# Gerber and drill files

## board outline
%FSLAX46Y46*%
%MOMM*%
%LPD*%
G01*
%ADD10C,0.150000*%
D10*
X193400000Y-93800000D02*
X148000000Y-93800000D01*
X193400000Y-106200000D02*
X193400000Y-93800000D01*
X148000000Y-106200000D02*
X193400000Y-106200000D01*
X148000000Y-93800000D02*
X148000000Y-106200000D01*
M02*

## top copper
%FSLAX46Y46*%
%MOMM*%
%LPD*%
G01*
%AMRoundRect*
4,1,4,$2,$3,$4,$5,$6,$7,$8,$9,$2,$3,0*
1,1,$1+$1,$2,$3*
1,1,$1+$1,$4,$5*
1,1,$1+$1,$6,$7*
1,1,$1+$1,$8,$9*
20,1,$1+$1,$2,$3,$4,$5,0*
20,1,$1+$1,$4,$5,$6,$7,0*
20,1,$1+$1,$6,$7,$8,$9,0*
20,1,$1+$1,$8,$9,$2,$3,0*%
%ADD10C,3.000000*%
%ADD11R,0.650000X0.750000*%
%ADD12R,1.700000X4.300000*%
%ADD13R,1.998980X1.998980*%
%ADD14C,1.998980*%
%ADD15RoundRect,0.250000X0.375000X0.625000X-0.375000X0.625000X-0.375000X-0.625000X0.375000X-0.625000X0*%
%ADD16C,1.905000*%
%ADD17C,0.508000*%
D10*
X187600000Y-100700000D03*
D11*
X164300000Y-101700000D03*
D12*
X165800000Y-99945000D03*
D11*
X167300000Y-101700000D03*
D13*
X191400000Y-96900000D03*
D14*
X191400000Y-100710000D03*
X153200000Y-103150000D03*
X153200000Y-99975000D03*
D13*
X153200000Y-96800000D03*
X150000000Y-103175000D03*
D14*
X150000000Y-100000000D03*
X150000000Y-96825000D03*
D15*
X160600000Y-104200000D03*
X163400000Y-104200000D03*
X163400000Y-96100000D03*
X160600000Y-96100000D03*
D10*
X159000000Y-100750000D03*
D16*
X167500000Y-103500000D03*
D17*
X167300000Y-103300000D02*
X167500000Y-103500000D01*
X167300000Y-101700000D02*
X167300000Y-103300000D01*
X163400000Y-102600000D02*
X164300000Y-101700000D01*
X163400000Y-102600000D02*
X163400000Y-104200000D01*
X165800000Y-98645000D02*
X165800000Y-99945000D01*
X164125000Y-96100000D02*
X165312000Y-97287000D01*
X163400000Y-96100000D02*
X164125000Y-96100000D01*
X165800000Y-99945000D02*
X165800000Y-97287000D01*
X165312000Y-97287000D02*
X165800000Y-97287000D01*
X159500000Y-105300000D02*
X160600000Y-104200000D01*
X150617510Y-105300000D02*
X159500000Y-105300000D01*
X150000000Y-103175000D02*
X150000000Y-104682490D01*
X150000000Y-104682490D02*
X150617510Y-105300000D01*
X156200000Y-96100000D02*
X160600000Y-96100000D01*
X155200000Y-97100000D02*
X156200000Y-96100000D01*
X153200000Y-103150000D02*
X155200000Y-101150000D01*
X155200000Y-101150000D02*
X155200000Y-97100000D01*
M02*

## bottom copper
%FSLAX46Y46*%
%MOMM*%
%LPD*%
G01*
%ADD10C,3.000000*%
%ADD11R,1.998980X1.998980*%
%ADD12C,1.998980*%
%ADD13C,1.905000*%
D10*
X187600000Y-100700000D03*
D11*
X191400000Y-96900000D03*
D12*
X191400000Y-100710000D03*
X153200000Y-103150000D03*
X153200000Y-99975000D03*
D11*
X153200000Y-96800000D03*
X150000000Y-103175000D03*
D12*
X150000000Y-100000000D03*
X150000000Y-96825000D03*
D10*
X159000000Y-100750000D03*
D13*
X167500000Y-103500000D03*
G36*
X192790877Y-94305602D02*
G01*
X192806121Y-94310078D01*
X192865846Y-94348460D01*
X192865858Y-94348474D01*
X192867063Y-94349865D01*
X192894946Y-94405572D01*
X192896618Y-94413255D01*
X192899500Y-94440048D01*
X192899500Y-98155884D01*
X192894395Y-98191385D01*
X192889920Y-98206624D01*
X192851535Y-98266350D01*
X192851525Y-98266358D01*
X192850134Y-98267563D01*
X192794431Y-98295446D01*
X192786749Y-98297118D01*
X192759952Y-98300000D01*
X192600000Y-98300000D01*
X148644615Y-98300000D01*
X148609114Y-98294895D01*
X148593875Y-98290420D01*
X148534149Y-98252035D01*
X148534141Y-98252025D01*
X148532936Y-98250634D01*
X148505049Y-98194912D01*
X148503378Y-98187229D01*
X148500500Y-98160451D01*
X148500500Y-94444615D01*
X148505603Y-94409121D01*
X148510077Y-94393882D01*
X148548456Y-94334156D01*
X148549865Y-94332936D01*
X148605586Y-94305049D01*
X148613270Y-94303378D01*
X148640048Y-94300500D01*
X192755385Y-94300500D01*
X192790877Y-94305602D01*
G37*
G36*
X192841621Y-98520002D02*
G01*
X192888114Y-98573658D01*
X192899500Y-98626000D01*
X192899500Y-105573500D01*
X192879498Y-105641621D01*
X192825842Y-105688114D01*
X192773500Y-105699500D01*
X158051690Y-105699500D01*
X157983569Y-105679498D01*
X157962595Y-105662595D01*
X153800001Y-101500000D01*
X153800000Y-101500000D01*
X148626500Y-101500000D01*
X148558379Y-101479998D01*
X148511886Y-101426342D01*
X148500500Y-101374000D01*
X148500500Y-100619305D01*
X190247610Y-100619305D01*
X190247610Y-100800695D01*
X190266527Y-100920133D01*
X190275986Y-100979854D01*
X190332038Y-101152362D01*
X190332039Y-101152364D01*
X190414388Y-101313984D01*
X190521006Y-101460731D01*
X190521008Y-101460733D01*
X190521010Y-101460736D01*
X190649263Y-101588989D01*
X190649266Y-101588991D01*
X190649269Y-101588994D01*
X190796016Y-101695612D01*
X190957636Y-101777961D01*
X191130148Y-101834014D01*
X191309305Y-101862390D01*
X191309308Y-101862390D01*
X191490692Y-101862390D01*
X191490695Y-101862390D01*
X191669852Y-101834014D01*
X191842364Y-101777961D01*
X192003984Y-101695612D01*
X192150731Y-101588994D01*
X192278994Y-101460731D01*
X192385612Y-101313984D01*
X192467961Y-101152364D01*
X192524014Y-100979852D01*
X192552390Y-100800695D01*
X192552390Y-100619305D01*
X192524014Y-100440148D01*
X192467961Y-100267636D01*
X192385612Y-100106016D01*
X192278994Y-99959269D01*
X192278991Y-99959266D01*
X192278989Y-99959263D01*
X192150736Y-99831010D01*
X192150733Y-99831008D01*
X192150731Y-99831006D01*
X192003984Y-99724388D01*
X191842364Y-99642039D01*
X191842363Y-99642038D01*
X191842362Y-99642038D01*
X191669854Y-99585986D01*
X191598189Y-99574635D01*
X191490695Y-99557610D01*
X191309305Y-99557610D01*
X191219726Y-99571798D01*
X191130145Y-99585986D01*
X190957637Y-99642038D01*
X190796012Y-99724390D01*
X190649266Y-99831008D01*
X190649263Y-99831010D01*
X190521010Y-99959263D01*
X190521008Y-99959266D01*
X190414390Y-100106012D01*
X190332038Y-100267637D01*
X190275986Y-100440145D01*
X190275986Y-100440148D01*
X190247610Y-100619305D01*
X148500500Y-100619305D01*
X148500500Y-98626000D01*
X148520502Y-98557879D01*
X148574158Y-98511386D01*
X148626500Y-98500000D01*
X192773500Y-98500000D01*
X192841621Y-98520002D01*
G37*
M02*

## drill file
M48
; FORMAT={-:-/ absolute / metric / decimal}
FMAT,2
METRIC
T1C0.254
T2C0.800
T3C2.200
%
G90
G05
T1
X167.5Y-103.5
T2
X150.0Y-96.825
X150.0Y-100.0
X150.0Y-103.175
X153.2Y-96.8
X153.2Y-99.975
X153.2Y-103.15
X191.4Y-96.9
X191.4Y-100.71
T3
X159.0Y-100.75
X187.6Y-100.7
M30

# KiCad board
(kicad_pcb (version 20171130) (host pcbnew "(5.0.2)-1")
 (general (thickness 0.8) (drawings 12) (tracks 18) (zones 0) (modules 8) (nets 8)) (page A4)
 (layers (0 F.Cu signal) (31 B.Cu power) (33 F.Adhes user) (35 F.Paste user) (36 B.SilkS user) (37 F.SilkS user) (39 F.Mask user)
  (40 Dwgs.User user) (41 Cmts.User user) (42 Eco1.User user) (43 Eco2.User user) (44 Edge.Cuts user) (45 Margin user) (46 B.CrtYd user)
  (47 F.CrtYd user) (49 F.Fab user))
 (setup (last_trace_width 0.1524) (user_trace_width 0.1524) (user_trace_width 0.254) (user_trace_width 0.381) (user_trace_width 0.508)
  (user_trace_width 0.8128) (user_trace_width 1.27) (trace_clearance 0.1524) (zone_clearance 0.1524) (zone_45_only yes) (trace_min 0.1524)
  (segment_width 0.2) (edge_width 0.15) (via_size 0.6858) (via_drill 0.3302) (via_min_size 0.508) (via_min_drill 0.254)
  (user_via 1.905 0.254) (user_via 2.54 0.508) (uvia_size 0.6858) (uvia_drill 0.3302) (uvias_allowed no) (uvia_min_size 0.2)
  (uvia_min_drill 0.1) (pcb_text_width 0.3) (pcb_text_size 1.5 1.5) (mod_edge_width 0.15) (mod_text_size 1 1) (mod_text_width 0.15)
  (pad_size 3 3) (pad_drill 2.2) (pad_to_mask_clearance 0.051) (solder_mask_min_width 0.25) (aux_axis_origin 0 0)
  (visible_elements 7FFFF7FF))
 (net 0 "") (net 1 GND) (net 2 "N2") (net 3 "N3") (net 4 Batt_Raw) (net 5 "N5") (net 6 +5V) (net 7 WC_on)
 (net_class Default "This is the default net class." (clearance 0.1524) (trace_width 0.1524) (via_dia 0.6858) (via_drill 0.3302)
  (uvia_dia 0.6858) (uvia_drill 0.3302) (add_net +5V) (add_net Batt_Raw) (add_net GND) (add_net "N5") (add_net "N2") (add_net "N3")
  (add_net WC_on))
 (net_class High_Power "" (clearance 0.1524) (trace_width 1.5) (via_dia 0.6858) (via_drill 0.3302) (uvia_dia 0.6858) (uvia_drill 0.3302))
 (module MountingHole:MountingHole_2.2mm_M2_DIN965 (layer F.Cu) (at 187.6 100.7)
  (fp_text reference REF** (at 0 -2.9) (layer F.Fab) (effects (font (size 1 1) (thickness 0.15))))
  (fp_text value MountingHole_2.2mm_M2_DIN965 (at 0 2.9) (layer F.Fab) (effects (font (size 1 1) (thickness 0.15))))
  (pad "" thru_hole circle (at 0 0) (size 3 3) (drill 2.2) (layers *.Cu *.Mask) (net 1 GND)))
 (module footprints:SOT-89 (layer F.Cu) (at 165.8 101.7)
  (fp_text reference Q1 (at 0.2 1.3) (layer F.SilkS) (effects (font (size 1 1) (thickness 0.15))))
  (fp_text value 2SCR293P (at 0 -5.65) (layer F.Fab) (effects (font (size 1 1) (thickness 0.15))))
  (pad 1 smd rect (at -1.5 0) (size 0.65 0.75) (layers F.Cu F.Paste F.Mask) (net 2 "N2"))
  (pad 2 smd rect (at 0 -1.755) (size 1.7 4.3) (layers F.Cu F.Paste F.Mask) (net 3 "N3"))
  (pad 3 smd rect (at 1.5 0) (size 0.65 0.75) (layers F.Cu F.Paste F.Mask) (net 1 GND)))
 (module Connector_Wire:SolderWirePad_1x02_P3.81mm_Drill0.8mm (layer F.Cu) (at 191.4 96.9 270)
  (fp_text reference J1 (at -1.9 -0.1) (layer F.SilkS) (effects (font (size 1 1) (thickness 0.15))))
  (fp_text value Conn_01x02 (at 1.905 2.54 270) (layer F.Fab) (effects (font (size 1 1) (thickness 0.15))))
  (pad 1 thru_hole rect (at 0 0 270) (size 1.99898 1.99898) (drill 0.8001) (layers *.Cu *.Mask) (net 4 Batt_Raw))
  (pad 2 thru_hole circle (at 3.81 0 270) (size 1.99898 1.99898) (drill 0.8001) (layers *.Cu *.Mask) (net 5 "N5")))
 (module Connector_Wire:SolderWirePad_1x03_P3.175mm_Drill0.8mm (layer F.Cu) (at 153.2 96.8 270)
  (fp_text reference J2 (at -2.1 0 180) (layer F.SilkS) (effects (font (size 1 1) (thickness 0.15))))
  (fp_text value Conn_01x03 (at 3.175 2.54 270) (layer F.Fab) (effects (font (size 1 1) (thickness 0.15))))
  (pad 3 thru_hole circle (at 6.35 0 270) (size 1.99898 1.99898) (drill 0.8001) (layers *.Cu *.Mask) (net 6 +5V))
  (pad 2 thru_hole circle (at 3.175 0 270) (size 1.99898 1.99898) (drill 0.8001) (layers *.Cu *.Mask) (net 1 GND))
  (pad 1 thru_hole rect (at 0 0 270) (size 1.99898 1.99898) (drill 0.8001) (layers *.Cu *.Mask) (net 4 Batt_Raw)))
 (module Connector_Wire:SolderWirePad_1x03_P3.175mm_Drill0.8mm (layer F.Cu) (at 150 103.175 90)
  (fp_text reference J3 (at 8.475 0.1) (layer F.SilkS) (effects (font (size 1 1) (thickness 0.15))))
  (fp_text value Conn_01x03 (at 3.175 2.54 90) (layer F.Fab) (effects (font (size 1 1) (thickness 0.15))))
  (pad 1 thru_hole rect (at 0 0 90) (size 1.99898 1.99898) (drill 0.8001) (layers *.Cu *.Mask) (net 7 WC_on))
  (pad 2 thru_hole circle (at 3.175 0 90) (size 1.99898 1.99898) (drill 0.8001) (layers *.Cu *.Mask) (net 1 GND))
  (pad 3 thru_hole circle (at 6.35 0 90) (size 1.99898 1.99898) (drill 0.8001) (layers *.Cu *.Mask) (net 4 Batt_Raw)))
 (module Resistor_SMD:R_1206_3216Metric (layer F.Cu) (at 162 104.2 180)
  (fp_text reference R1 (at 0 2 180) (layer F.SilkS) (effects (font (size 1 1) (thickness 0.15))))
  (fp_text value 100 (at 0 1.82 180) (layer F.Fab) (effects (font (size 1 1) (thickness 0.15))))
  (pad 2 smd roundrect (at 1.4 0 180) (size 1.25 1.75) (layers F.Cu F.Paste F.Mask) (roundrect_rratio 0.2) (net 7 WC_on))
  (pad 1 smd roundrect (at -1.4 0 180) (size 1.25 1.75) (layers F.Cu F.Paste F.Mask) (roundrect_rratio 0.2) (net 2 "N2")))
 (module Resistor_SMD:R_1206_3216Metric (layer F.Cu) (at 162 96.1 180)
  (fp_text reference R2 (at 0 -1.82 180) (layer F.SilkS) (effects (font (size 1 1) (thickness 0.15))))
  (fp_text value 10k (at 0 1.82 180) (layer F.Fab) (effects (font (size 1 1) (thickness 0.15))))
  (pad 1 smd roundrect (at -1.4 0 180) (size 1.25 1.75) (layers F.Cu F.Paste F.Mask) (roundrect_rratio 0.2) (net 3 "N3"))
  (pad 2 smd roundrect (at 1.4 0 180) (size 1.25 1.75) (layers F.Cu F.Paste F.Mask) (roundrect_rratio 0.2) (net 6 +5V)))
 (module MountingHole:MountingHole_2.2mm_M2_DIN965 (layer F.Cu) (at 159 100.75)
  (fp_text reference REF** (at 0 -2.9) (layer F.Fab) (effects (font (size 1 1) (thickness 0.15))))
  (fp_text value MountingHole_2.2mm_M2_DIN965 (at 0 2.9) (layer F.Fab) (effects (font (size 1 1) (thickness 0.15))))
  (pad "" thru_hole circle (at 0 0) (size 3 3) (drill 2.2) (layers *.Cu *.Mask) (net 1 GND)))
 (gr_line (start 193.4 93.8) (end 148 93.8) (layer Edge.Cuts) (width 0.15))
 (gr_line (start 193.4 106.2) (end 193.4 93.8) (layer Edge.Cuts) (width 0.15))
 (gr_line (start 148 106.2) (end 193.4 106.2) (layer Edge.Cuts) (width 0.15))
 (gr_line (start 148 93.8) (end 148 106.2) (layer Edge.Cuts) (width 0.15))
 (via (at 167.5 103.5) (size 1.905) (drill 0.254) (layers F.Cu B.Cu) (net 1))
 (segment (start 167.3 103.3) (end 167.5 103.5) (width 0.508) (layer F.Cu) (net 1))
 (segment (start 167.3 101.7) (end 167.3 103.3) (width 0.508) (layer F.Cu) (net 1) (status 10))
 (segment (start 163.4 102.6) (end 164.3 101.7) (width 0.508) (layer F.Cu) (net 2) (status 20))
 (segment (start 163.4 102.6) (end 163.4 104.2) (width 0.508) (layer F.Cu) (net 2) (status 20))
 (segment (start 165.8 98.645) (end 165.8 99.945) (width 0.508) (layer F.Cu) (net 3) (status 30))
 (segment (start 164.125 96.1) (end 165.312 97.287) (width 0.508) (layer F.Cu) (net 3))
 (segment (start 163.4 96.1) (end 164.125 96.1) (width 0.508) (layer F.Cu) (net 3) (status 10))
 (segment (start 165.8 99.945) (end 165.8 97.287) (width 0.508) (layer F.Cu) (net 3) (status 10))
 (segment (start 165.312 97.287) (end 165.8 97.287) (width 0.508) (layer F.Cu) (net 3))
 (segment (start 159.5 105.3) (end 160.6 104.2) (width 0.508) (layer F.Cu) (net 7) (status 20))
 (segment (start 150.61751 105.3) (end 159.5 105.3) (width 0.508) (layer F.Cu) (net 7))
 (segment (start 150 103.175) (end 150 104.68249) (width 0.508) (layer F.Cu) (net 7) (status 10))
 (segment (start 150 104.68249) (end 150.61751 105.3) (width 0.508) (layer F.Cu) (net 7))
 (segment (start 156.2 96.1) (end 160.6 96.1) (width 0.508) (layer F.Cu) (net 6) (status 20))
 (segment (start 155.2 97.1) (end 156.2 96.1) (width 0.508) (layer F.Cu) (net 6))
 (segment (start 153.2 103.15) (end 155.2 101.15) (width 0.508) (layer F.Cu) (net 6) (status 10))
 (segment (start 155.2 101.15) (end 155.2 97.1) (width 0.508) (layer F.Cu) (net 6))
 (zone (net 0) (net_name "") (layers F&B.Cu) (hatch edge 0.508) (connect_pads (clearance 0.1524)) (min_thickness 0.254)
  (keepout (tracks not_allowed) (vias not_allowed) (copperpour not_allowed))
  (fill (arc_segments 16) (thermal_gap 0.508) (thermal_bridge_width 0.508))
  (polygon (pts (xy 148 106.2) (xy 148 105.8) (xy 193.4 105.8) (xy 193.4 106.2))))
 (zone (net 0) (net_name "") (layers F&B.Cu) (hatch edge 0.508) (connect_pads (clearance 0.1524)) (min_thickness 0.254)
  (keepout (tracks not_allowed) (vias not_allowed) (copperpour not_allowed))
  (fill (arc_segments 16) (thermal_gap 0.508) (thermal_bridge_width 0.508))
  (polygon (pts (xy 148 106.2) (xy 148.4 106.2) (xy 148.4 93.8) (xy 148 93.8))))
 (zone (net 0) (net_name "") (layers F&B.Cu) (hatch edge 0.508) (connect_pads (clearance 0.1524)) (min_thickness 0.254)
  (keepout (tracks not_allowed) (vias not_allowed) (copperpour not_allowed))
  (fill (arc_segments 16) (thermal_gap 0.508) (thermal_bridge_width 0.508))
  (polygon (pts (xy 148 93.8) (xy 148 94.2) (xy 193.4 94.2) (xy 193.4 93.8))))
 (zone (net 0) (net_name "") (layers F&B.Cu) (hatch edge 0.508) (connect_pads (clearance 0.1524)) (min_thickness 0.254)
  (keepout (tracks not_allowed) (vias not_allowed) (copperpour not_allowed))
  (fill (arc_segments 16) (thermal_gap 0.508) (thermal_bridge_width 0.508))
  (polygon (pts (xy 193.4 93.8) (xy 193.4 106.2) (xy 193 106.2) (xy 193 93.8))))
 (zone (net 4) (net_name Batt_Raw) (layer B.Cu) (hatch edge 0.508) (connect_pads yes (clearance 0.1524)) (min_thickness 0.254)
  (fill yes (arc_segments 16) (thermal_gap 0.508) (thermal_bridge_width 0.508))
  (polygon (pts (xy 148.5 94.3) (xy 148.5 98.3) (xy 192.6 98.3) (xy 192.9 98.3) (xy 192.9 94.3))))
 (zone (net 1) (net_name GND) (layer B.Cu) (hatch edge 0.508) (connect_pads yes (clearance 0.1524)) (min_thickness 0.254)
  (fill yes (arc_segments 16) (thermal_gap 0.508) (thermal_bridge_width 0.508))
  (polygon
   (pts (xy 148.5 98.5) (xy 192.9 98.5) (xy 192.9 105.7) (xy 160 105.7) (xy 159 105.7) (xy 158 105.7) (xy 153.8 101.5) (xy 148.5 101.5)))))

